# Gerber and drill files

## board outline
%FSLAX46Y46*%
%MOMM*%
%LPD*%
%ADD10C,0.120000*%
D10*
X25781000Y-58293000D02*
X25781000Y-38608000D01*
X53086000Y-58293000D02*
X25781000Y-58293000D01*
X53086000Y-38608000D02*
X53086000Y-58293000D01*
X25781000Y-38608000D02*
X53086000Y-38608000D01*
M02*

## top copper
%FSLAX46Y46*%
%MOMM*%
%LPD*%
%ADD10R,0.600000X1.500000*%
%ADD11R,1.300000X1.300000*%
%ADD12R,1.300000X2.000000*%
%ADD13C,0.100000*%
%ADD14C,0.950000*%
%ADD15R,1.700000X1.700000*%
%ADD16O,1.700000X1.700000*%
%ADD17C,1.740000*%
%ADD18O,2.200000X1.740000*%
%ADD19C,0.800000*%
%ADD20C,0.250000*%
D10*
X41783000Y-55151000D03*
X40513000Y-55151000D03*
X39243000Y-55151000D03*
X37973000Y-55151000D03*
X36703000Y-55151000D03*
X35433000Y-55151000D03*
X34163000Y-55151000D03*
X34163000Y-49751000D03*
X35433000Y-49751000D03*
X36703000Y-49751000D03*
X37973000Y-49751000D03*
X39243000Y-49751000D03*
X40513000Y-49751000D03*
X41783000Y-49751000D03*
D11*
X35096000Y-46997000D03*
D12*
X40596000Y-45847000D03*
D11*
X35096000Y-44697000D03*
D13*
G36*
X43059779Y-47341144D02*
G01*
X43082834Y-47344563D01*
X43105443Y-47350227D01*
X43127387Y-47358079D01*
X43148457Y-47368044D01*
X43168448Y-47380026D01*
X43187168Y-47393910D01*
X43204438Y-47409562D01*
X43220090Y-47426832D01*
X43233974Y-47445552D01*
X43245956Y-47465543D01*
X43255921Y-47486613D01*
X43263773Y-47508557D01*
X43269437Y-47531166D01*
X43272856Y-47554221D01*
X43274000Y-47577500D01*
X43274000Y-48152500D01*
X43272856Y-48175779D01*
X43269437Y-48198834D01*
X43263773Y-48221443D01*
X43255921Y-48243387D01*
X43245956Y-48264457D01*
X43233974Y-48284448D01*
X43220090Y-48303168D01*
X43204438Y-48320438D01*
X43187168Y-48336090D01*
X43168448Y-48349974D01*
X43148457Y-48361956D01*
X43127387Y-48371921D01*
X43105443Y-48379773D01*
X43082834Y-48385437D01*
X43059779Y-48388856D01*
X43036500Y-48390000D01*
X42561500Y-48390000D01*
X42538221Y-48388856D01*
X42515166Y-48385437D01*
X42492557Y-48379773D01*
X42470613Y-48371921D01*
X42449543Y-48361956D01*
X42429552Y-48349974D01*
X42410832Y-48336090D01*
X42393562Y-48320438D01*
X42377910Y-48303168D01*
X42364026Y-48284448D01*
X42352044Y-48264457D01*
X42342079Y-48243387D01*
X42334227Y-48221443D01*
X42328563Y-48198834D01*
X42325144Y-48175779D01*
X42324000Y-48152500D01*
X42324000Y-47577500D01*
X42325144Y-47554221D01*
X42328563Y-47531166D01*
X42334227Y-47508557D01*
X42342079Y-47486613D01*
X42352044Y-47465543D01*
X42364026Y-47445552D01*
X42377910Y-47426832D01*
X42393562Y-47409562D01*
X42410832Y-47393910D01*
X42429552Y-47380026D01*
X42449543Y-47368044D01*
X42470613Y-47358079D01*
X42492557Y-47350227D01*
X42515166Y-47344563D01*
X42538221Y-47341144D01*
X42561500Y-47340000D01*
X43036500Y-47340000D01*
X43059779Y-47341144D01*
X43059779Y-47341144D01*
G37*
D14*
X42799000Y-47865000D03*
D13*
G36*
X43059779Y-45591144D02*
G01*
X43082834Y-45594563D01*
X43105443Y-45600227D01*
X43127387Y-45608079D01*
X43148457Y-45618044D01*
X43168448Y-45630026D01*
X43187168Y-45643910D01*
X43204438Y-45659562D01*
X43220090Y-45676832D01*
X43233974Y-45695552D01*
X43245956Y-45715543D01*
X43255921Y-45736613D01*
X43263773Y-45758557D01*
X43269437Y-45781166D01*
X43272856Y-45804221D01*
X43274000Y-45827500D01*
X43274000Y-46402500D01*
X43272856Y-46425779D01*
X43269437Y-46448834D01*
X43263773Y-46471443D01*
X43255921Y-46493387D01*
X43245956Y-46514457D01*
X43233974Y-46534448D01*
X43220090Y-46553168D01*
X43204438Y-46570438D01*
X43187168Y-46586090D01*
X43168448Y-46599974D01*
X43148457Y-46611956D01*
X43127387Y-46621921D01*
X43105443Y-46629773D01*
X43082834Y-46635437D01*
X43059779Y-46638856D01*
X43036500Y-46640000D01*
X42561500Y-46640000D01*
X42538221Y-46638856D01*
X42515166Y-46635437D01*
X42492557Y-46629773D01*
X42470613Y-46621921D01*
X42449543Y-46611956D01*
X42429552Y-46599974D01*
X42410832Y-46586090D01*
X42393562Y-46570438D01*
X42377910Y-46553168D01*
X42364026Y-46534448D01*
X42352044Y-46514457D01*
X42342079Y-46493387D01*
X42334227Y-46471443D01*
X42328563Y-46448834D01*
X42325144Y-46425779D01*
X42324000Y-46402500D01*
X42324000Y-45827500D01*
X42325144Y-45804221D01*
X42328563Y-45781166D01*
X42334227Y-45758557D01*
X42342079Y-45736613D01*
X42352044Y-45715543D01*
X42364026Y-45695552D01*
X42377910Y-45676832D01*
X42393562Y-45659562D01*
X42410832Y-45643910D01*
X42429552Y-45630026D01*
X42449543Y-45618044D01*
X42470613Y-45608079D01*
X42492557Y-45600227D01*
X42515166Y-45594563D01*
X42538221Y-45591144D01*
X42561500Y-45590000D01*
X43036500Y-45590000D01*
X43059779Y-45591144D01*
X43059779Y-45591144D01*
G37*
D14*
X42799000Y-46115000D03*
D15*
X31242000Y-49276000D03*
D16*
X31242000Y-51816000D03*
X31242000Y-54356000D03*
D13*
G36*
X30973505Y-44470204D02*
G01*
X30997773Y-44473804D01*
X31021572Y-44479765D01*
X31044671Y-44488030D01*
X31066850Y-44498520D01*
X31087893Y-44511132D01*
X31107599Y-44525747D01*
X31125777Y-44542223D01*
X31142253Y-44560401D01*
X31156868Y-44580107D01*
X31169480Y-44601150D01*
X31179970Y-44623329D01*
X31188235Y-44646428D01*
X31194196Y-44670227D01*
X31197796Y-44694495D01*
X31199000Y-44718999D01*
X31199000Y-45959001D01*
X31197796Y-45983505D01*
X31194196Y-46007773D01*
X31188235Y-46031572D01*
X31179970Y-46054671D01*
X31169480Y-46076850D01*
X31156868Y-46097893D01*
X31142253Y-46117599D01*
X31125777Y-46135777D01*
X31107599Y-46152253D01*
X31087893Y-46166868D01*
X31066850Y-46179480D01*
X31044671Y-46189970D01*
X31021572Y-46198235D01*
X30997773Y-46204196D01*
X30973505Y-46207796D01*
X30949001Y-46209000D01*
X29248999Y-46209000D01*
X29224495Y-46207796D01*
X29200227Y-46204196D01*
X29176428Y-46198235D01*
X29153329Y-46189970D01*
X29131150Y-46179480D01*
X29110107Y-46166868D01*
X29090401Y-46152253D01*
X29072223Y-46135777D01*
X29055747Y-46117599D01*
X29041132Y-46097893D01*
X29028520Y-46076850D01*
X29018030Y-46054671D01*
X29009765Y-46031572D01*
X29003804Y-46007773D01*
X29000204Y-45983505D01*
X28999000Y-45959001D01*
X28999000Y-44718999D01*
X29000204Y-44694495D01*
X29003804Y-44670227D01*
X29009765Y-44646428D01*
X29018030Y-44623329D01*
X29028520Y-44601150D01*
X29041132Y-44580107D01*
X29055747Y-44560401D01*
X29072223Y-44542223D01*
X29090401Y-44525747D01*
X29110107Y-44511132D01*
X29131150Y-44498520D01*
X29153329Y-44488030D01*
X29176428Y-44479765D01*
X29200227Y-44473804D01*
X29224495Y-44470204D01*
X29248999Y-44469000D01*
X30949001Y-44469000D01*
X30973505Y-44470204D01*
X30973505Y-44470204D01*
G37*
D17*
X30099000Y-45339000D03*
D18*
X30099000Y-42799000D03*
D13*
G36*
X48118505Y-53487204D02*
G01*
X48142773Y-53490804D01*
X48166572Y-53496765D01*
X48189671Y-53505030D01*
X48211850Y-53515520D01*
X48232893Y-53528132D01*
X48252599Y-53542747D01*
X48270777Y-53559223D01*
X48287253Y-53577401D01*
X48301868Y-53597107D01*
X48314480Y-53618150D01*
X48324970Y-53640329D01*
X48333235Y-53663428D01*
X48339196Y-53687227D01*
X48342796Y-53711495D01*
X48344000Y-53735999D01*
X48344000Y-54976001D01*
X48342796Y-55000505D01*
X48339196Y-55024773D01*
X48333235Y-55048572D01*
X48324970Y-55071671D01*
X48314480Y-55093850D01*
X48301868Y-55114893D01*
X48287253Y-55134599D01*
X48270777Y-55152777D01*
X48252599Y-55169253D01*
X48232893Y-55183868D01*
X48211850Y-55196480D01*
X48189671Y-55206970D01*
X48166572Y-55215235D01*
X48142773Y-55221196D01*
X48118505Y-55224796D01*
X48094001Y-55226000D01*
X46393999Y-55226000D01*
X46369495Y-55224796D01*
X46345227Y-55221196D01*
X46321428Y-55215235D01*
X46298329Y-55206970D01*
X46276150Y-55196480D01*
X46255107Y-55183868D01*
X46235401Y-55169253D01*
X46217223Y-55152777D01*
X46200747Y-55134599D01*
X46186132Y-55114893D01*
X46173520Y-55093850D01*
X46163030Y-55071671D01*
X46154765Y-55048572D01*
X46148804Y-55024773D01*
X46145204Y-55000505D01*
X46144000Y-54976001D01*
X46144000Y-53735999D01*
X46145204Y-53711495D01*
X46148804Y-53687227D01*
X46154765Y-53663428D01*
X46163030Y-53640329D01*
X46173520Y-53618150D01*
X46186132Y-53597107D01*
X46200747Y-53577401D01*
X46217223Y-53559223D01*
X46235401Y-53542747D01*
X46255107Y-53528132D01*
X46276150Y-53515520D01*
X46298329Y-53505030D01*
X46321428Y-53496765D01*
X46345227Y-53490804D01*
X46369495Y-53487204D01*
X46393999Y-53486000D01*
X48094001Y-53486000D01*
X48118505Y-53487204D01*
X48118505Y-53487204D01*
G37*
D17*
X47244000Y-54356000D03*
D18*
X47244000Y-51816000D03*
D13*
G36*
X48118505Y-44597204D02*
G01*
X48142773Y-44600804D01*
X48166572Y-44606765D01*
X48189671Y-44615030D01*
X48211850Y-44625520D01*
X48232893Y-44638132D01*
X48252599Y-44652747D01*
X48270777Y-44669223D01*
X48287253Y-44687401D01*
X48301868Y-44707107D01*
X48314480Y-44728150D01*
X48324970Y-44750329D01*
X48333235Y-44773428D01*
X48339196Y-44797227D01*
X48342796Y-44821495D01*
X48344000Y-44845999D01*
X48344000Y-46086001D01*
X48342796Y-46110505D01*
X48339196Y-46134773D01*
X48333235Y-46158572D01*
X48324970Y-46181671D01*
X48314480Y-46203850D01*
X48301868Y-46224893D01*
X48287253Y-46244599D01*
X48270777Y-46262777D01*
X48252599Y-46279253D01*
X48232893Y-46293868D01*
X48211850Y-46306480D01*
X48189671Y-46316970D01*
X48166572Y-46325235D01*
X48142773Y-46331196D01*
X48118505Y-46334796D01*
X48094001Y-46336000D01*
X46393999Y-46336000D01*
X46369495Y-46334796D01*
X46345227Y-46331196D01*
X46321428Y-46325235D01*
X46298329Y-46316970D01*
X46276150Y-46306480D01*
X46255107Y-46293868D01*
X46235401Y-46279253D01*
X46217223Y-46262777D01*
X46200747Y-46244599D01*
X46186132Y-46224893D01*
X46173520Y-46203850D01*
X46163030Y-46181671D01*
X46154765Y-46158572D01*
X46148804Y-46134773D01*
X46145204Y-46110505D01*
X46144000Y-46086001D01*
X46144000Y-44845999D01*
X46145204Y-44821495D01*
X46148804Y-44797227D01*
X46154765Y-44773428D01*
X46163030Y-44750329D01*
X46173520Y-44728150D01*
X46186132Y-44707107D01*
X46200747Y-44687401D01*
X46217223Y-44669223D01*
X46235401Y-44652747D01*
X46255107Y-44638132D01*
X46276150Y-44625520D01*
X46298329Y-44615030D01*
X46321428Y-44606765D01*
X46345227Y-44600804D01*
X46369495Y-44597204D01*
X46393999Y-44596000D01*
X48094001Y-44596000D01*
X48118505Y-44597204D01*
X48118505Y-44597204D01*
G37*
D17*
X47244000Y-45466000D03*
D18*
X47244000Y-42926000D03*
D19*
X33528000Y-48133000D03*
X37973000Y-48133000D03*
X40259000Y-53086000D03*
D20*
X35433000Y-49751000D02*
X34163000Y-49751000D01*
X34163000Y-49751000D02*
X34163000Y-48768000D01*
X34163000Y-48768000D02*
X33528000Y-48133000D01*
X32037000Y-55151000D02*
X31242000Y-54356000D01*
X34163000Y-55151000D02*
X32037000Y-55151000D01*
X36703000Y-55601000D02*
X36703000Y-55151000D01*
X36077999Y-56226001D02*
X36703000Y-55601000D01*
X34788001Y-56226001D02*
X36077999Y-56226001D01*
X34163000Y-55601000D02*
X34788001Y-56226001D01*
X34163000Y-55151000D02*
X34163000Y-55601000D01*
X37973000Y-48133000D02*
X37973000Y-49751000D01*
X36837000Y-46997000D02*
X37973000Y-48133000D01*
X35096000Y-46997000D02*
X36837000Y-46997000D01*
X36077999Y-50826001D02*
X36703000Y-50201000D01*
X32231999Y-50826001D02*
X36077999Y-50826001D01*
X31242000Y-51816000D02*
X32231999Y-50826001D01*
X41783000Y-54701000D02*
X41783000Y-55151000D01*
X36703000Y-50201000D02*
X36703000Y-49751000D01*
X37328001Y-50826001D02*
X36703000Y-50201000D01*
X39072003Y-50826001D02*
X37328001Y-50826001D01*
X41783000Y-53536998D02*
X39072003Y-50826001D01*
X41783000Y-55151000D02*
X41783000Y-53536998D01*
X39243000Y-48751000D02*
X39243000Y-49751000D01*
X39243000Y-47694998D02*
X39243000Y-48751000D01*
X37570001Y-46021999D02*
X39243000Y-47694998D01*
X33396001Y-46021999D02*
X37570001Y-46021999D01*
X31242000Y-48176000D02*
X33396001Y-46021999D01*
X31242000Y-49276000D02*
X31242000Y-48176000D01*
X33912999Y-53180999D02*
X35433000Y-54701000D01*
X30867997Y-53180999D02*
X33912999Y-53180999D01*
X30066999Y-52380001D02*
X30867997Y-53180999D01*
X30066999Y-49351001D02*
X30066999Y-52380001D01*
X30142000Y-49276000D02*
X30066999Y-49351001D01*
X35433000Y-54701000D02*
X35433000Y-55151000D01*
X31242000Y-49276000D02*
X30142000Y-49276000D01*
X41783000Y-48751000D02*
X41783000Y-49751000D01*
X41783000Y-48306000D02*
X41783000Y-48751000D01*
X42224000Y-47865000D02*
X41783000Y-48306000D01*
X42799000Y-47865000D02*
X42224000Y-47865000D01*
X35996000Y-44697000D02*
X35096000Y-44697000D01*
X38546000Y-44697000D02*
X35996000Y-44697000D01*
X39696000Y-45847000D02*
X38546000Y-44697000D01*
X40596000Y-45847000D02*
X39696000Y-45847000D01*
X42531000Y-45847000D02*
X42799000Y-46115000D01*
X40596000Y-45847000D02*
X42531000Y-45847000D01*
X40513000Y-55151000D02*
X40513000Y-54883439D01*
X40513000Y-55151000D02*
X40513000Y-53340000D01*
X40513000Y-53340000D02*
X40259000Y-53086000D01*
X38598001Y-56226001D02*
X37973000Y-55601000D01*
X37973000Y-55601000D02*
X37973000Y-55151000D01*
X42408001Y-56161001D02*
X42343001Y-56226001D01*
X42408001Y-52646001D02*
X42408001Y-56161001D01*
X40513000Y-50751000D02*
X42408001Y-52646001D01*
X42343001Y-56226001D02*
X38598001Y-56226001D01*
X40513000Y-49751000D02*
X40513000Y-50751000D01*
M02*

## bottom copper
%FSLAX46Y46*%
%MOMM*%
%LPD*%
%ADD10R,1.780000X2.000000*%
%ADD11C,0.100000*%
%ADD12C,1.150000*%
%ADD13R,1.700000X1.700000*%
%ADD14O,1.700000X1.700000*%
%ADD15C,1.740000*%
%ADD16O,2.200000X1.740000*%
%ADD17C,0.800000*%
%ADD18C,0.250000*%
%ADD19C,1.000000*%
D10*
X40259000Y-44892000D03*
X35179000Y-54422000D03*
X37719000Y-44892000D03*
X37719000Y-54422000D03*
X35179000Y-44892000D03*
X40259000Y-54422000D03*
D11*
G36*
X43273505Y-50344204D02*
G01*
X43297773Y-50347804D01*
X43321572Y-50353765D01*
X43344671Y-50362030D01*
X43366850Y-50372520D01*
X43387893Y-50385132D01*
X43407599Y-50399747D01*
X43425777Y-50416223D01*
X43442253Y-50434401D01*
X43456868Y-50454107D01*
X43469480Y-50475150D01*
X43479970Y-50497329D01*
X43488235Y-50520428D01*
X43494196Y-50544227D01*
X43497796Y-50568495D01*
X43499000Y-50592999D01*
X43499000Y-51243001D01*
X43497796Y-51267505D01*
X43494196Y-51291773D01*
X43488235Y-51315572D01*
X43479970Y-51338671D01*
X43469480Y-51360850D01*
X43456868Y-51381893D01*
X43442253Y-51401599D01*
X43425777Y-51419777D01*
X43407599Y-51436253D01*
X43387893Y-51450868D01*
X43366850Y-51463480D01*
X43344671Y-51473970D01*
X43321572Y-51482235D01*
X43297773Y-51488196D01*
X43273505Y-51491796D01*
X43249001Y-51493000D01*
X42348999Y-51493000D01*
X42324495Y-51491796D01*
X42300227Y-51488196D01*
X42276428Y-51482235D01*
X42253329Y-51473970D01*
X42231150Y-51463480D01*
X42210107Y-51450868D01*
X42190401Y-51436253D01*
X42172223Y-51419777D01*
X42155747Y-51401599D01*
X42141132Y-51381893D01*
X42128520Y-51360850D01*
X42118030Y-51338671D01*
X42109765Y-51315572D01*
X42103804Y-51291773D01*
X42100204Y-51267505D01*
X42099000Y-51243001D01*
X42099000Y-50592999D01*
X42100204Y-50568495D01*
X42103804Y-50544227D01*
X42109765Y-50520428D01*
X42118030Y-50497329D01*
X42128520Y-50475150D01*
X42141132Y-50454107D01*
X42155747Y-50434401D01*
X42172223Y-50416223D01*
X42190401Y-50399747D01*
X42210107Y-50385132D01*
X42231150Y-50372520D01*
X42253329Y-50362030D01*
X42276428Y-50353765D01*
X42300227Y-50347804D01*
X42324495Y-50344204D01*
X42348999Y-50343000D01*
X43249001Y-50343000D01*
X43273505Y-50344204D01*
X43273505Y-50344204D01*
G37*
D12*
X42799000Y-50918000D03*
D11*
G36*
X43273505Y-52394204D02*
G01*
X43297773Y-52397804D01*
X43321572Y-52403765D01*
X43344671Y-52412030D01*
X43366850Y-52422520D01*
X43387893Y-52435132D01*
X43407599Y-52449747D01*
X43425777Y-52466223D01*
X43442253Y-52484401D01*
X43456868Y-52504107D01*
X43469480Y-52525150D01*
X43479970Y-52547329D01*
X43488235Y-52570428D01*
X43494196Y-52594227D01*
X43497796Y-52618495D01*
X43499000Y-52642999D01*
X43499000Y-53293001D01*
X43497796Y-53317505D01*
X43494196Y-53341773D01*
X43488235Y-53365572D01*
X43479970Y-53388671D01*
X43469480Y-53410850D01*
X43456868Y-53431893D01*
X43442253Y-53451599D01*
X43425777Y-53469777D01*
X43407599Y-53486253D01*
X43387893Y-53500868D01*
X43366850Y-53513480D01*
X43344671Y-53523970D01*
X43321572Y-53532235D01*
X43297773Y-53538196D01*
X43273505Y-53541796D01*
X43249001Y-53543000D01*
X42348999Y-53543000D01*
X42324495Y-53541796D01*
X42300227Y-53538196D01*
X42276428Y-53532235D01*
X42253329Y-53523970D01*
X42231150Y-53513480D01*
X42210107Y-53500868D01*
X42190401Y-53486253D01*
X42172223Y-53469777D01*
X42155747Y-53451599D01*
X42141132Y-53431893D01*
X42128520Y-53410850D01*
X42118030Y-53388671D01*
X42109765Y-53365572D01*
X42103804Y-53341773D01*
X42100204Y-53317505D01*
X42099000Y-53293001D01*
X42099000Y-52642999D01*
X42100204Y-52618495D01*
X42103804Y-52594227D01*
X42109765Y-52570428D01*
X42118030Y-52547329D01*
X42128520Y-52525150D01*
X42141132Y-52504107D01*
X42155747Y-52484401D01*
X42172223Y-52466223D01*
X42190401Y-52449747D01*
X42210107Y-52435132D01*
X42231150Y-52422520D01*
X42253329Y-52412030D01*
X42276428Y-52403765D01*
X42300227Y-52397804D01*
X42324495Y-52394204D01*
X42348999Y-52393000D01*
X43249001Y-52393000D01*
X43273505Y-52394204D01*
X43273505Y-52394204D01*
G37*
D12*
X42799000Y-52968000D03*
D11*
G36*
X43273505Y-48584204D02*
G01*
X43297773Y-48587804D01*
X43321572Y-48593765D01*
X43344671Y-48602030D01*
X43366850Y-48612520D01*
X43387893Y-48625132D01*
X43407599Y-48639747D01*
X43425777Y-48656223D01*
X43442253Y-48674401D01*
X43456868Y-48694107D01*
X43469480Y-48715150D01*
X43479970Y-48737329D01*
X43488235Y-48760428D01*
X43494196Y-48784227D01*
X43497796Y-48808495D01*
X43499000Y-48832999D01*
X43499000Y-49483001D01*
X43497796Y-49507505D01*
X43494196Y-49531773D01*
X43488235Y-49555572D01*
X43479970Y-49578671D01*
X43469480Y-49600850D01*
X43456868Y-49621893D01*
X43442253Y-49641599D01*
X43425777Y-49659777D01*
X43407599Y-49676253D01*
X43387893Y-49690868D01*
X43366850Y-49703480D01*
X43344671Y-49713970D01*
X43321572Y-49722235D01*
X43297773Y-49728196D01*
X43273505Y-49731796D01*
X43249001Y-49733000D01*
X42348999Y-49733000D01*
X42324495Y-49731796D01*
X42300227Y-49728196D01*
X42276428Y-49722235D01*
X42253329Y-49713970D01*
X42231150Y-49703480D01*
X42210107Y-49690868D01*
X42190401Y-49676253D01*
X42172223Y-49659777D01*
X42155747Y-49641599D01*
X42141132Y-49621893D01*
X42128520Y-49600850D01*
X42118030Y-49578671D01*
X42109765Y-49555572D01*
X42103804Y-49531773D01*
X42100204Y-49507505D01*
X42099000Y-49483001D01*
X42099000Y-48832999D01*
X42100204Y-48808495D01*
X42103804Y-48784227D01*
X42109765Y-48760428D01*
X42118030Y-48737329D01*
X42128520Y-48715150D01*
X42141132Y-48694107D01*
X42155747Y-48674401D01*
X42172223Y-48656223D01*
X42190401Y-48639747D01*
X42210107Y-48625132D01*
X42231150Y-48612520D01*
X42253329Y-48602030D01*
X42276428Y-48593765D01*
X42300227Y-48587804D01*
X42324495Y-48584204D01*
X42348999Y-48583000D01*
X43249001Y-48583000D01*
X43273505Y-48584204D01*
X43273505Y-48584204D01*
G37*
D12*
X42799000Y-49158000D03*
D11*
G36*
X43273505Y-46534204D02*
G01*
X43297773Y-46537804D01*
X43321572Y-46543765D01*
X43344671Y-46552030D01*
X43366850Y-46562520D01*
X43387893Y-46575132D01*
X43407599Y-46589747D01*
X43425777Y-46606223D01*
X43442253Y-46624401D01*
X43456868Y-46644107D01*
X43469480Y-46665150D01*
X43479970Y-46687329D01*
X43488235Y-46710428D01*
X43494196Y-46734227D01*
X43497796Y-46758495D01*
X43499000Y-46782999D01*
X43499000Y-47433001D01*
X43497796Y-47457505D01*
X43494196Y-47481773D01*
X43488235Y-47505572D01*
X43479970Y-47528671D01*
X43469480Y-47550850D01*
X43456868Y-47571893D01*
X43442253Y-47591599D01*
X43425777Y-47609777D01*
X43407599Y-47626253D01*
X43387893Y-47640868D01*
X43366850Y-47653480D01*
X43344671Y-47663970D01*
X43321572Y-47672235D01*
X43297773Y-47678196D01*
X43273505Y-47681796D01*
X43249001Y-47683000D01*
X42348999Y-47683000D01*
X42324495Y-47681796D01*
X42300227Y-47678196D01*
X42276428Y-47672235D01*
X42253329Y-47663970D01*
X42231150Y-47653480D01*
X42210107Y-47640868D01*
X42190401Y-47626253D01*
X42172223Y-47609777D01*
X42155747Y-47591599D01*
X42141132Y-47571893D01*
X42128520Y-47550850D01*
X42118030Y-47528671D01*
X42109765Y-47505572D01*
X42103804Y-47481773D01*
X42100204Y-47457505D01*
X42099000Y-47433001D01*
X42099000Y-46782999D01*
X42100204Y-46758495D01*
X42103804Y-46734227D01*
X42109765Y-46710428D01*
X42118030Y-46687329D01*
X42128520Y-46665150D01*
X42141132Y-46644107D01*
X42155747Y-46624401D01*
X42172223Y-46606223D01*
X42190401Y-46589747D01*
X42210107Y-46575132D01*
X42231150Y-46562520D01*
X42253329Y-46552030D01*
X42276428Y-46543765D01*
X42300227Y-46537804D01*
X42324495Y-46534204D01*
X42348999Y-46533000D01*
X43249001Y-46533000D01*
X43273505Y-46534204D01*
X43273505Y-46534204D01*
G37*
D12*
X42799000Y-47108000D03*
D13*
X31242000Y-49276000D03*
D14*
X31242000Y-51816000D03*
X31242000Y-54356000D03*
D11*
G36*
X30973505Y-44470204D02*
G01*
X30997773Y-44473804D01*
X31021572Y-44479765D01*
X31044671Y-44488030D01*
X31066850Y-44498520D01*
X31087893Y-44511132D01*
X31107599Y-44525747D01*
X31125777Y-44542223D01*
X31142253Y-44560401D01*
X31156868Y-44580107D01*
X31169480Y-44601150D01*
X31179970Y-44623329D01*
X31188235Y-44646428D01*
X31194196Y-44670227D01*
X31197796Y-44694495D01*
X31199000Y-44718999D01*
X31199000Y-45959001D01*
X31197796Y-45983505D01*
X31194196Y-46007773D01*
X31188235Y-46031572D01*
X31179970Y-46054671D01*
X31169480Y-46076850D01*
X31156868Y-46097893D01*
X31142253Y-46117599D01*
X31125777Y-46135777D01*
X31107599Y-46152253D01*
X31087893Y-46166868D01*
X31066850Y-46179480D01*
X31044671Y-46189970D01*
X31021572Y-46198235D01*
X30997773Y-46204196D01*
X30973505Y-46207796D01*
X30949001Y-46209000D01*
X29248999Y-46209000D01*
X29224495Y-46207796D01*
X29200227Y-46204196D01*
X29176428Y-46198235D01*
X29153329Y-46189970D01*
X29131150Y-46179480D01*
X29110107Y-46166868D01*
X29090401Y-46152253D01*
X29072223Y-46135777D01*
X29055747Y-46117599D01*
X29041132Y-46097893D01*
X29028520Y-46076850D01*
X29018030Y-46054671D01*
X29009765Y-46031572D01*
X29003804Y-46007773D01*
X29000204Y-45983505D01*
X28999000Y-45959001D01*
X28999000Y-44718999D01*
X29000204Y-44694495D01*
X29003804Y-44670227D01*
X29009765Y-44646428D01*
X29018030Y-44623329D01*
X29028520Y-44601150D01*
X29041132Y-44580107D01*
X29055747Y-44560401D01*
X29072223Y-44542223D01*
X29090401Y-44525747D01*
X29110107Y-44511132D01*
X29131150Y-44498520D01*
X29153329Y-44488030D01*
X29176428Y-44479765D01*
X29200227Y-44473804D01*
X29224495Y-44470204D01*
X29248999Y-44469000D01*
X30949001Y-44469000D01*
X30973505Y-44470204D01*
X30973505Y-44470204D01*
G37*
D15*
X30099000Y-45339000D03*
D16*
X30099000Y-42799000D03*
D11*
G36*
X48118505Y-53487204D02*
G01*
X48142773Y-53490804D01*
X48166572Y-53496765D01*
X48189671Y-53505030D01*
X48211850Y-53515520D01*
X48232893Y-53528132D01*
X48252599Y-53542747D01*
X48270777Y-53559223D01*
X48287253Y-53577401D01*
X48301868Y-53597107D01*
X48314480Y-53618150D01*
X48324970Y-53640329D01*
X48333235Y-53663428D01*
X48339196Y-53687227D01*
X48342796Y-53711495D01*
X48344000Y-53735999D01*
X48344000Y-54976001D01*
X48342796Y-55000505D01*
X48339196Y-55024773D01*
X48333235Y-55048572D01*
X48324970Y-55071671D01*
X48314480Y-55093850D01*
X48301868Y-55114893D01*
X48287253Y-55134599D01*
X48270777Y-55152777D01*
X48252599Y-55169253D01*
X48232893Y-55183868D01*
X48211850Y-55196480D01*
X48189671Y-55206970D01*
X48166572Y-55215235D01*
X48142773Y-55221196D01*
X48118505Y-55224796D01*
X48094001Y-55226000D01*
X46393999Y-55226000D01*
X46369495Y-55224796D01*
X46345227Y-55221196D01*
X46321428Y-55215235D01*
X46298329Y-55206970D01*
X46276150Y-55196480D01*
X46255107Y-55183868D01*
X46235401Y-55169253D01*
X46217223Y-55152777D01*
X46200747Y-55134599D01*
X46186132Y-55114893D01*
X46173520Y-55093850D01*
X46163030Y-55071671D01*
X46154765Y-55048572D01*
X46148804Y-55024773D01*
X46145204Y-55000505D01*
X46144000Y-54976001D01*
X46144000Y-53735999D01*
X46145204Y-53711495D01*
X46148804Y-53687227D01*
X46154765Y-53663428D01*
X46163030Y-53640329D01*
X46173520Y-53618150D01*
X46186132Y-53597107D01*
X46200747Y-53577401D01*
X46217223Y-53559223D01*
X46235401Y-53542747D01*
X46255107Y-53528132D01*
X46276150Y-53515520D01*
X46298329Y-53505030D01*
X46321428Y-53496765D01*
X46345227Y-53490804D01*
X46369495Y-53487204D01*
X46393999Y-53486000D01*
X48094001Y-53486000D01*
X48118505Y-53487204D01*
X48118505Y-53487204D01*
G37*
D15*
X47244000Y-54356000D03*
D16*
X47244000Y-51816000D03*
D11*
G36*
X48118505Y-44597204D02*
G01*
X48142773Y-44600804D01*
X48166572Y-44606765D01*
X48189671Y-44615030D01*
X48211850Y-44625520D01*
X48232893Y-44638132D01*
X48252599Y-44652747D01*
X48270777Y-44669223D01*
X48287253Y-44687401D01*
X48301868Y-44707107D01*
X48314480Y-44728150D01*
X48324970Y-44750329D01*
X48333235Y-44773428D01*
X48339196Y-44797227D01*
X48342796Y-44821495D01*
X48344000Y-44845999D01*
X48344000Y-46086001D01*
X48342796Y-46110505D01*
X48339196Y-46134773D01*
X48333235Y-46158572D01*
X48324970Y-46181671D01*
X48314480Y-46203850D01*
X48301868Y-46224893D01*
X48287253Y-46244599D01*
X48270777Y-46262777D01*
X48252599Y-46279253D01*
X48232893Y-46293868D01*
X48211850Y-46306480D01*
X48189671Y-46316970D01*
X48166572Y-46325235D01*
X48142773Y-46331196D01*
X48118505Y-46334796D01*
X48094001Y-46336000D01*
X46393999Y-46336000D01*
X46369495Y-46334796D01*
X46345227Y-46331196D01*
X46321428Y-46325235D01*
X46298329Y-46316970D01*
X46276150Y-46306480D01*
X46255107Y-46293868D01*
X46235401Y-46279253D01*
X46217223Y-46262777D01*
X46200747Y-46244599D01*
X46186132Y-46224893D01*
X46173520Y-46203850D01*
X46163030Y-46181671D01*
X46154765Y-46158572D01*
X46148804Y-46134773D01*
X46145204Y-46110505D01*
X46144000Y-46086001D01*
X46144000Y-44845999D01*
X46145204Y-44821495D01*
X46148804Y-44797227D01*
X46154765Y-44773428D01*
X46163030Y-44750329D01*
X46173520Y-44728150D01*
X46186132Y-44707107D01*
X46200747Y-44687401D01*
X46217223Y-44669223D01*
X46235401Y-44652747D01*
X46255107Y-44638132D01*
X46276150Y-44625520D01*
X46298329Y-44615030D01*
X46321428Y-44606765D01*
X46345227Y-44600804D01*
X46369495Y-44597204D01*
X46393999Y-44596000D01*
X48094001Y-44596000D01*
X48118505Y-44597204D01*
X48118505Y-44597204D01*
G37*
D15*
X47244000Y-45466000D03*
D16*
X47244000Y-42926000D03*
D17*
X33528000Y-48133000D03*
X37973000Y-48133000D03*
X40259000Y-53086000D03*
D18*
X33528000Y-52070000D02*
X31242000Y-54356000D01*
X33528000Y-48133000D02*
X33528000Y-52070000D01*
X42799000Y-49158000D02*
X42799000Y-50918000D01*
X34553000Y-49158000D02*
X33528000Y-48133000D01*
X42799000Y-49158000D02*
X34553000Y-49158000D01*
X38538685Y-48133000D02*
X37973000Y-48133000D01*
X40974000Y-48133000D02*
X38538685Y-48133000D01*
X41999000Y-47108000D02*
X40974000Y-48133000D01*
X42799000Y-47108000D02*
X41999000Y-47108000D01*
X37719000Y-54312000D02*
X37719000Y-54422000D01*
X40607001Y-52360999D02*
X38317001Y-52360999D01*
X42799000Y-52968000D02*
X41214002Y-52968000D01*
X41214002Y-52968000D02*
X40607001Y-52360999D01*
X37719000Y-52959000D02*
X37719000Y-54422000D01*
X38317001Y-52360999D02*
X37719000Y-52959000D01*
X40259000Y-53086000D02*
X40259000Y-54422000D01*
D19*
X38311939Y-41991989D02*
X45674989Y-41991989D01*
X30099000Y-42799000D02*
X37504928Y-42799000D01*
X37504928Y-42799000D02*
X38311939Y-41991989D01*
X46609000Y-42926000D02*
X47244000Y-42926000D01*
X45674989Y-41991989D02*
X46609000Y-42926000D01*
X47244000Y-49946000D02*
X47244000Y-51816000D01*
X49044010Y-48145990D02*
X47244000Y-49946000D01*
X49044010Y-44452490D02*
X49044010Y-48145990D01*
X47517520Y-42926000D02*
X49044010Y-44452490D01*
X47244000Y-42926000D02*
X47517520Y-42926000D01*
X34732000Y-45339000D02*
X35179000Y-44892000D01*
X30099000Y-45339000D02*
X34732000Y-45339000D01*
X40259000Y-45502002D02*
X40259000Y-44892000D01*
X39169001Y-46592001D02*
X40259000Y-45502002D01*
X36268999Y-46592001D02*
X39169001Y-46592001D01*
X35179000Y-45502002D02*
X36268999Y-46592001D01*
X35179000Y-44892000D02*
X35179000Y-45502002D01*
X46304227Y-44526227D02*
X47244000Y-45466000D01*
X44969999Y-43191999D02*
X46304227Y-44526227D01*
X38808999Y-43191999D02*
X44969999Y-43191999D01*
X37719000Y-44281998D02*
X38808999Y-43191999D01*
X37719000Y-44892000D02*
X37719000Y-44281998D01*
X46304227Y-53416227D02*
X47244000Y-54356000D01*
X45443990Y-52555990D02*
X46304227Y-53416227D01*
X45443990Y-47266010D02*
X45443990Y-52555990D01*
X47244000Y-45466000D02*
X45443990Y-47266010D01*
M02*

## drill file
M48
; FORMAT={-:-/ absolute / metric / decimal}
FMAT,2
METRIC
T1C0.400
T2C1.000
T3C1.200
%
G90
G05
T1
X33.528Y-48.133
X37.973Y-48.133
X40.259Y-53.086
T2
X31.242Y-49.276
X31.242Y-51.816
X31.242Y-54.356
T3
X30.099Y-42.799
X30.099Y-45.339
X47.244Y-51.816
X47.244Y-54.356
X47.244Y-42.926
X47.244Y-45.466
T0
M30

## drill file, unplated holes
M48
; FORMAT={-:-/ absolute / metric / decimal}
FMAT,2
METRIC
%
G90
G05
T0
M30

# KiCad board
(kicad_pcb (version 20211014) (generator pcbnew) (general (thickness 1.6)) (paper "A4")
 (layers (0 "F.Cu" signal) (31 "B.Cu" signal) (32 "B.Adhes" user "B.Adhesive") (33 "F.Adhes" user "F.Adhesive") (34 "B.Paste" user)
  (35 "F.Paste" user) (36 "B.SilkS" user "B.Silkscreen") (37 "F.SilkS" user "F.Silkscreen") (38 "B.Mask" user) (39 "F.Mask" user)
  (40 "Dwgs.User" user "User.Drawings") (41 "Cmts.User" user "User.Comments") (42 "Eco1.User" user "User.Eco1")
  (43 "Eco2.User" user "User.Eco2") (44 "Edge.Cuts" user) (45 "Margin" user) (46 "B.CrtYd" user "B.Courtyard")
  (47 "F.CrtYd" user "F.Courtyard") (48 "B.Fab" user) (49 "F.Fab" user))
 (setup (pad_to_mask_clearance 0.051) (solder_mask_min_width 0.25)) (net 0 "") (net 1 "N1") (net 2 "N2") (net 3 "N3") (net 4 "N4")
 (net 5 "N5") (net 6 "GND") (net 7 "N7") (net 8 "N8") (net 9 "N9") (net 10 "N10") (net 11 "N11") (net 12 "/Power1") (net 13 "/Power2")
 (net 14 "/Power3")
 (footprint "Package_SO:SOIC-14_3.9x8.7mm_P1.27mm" (layer "F.Cu") (at 37.973 52.451 -90)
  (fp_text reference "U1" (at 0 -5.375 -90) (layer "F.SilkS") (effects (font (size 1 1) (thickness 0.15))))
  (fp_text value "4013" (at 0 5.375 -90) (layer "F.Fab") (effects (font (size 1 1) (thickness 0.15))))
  (pad "1" smd rect locked (at -2.7 -3.81 270) (size 1.5 0.6) (layers "F.Cu" "F.Paste" "F.Mask") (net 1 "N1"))
  (pad "2" smd rect locked (at -2.7 -2.54 270) (size 1.5 0.6) (layers "F.Cu" "F.Paste" "F.Mask") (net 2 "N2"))
  (pad "3" smd rect locked (at -2.7 -1.27 270) (size 1.5 0.6) (layers "F.Cu" "F.Paste" "F.Mask") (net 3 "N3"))
  (pad "4" smd rect locked (at -2.7 0 270) (size 1.5 0.6) (layers "F.Cu" "F.Paste" "F.Mask") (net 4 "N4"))
  (pad "5" smd rect locked (at -2.7 1.27 270) (size 1.5 0.6) (layers "F.Cu" "F.Paste" "F.Mask") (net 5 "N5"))
  (pad "6" smd rect locked (at -2.7 2.54 270) (size 1.5 0.6) (layers "F.Cu" "F.Paste" "F.Mask") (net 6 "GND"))
  (pad "7" smd rect locked (at -2.7 3.81 270) (size 1.5 0.6) (layers "F.Cu" "F.Paste" "F.Mask") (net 6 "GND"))
  (pad "8" smd rect locked (at 2.7 3.81 270) (size 1.5 0.6) (layers "F.Cu" "F.Paste" "F.Mask") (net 6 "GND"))
  (pad "9" smd rect locked (at 2.7 2.54 270) (size 1.5 0.6) (layers "F.Cu" "F.Paste" "F.Mask") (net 3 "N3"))
  (pad "10" smd rect locked (at 2.7 1.27 270) (size 1.5 0.6) (layers "F.Cu" "F.Paste" "F.Mask") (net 6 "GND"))
  (pad "11" smd rect locked (at 2.7 0 270) (size 1.5 0.6) (layers "F.Cu" "F.Paste" "F.Mask") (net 2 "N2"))
  (pad "12" smd rect locked (at 2.7 -1.27 270) (size 1.5 0.6) (layers "F.Cu" "F.Paste" "F.Mask") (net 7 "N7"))
  (pad "13" smd rect locked (at 2.7 -2.54 270) (size 1.5 0.6) (layers "F.Cu" "F.Paste" "F.Mask") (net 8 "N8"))
  (pad "14" smd rect locked (at 2.7 -3.81 270) (size 1.5 0.6) (layers "F.Cu" "F.Paste" "F.Mask") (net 5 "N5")))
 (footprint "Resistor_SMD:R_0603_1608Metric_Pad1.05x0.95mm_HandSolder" (layer "F.Cu") (at 42.799 46.99 -90)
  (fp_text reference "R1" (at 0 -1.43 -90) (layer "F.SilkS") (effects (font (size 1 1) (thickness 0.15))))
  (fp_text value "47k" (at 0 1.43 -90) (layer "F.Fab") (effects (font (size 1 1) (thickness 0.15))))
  (pad "1" smd roundrect locked (at -0.875 0 270) (size 1.05 0.95) (layers "F.Cu" "F.Paste" "F.Mask") (roundrect_rratio 0.25) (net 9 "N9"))
  (pad "2" smd roundrect locked (at 0.875 0 270) (size 1.05 0.95) (layers "F.Cu" "F.Paste" "F.Mask") (roundrect_rratio 0.25) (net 1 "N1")))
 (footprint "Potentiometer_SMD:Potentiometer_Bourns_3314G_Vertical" (layer "F.Cu") (at 37.846 45.847 90)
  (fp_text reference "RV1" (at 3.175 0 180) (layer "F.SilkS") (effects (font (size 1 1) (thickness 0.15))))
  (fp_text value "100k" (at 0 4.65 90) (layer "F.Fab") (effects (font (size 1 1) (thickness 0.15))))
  (pad "1" smd rect locked (at 1.15 -2.75 90) (size 1.3 1.3) (layers "F.Cu" "F.Paste" "F.Mask") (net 9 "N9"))
  (pad "2" smd rect locked (at 0 2.75 90) (size 2 1.3) (layers "F.Cu" "F.Paste" "F.Mask") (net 9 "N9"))
  (pad "3" smd rect locked (at -1.15 -2.75 90) (size 1.3 1.3) (layers "F.Cu" "F.Paste" "F.Mask") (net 4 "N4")))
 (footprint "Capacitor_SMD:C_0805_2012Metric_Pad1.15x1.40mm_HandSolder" (layer "B.Cu") (at 42.799 48.133 -90)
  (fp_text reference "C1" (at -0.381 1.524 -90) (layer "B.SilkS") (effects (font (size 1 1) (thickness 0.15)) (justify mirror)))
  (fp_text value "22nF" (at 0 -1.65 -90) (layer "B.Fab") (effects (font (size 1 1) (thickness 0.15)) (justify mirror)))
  (pad "1" smd roundrect locked (at -1.025 0 270) (size 1.15 1.4) (layers "B.Cu" "B.Paste" "B.Mask") (roundrect_rratio 0.217391)
   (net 4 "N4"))
  (pad "2" smd roundrect locked (at 1.025 0 270) (size 1.15 1.4) (layers "B.Cu" "B.Paste" "B.Mask") (roundrect_rratio 0.217391)
   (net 6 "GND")))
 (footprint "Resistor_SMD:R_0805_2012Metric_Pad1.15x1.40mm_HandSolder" (layer "B.Cu") (at 42.799 51.943 90)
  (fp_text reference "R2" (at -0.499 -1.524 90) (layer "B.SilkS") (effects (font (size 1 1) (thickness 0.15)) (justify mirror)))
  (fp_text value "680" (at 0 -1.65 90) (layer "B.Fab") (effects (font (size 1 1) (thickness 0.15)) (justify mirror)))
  (pad "1" smd roundrect locked (at -1.025 0 90) (size 1.15 1.4) (layers "B.Cu" "B.Paste" "B.Mask") (roundrect_rratio 0.217391)
   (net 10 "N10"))
  (pad "2" smd roundrect locked (at 1.025 0 90) (size 1.15 1.4) (layers "B.Cu" "B.Paste" "B.Mask") (roundrect_rratio 0.217391) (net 6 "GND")))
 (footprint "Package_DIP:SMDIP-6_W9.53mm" (layer "B.Cu") (at 37.719 49.657 90)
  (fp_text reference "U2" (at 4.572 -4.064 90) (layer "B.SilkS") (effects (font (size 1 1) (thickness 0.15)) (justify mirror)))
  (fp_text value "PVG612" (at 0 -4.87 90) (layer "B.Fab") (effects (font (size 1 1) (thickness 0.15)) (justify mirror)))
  (pad "1" smd rect locked (at -4.765 2.54 90) (size 2 1.78) (layers "B.Cu" "B.Paste" "B.Mask") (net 8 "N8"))
  (pad "2" smd rect locked (at -4.765 0 90) (size 2 1.78) (layers "B.Cu" "B.Paste" "B.Mask") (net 10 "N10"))
  (pad "3" smd rect locked (at -4.765 -2.54 90) (size 2 1.78) (layers "B.Cu" "B.Paste" "B.Mask") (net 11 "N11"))
  (pad "4" smd rect locked (at 4.765 -2.54 90) (size 2 1.78) (layers "B.Cu" "B.Paste" "B.Mask") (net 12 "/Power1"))
  (pad "5" smd rect locked (at 4.765 0 90) (size 2 1.78) (layers "B.Cu" "B.Paste" "B.Mask") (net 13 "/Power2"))
  (pad "6" smd rect locked (at 4.765 2.54 90) (size 2 1.78) (layers "B.Cu" "B.Paste" "B.Mask") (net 12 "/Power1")))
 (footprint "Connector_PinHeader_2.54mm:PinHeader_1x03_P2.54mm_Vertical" (layer "B.Cu") (at 31.242 49.276 180)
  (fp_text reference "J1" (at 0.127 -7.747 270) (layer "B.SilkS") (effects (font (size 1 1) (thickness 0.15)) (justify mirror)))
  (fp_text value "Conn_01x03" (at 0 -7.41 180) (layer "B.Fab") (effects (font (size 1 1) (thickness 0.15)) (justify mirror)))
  (pad "1" thru_hole rect locked (at 0 0 180) (size 1.7 1.7) (drill 1) (layers *.Cu *.Mask) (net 3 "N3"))
  (pad "2" thru_hole oval locked (at 0 -2.54 180) (size 1.7 1.7) (drill 1) (layers *.Cu *.Mask) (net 5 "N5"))
  (pad "3" thru_hole oval locked (at 0 -5.08 180) (size 1.7 1.7) (drill 1) (layers *.Cu *.Mask) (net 6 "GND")))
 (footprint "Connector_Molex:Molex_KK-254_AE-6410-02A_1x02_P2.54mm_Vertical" (layer "B.Cu") (at 30.099 45.339 90)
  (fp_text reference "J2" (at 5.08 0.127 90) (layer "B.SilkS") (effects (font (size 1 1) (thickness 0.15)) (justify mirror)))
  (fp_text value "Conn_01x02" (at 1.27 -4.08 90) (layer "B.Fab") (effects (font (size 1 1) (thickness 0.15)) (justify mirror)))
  (pad "1" thru_hole roundrect locked (at 0 0 90) (size 1.74 2.2) (drill 1.2) (layers *.Cu *.Mask) (roundrect_rratio 0.143678)
   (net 12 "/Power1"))
  (pad "2" thru_hole oval locked (at 2.54 0 90) (size 1.74 2.2) (drill 1.2) (layers *.Cu *.Mask) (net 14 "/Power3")))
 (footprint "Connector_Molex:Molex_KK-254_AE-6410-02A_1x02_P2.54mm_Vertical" (layer "B.Cu") (at 47.244 54.356 90)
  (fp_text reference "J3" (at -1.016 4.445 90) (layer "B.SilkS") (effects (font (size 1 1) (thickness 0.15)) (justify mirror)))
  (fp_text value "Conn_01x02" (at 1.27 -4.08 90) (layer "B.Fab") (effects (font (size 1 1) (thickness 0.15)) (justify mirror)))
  (pad "1" thru_hole roundrect locked (at 0 0 90) (size 1.74 2.2) (drill 1.2) (layers *.Cu *.Mask) (roundrect_rratio 0.143678)
   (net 13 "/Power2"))
  (pad "2" thru_hole oval locked (at 2.54 0 90) (size 1.74 2.2) (drill 1.2) (layers *.Cu *.Mask) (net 14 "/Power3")))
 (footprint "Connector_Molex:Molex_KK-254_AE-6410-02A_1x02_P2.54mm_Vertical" (layer "B.Cu") (at 47.244 45.466 90)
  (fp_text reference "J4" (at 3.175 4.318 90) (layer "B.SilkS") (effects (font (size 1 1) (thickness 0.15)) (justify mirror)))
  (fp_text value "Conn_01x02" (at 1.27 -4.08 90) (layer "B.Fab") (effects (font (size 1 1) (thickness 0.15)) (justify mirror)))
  (pad "1" thru_hole roundrect locked (at 0 0 90) (size 1.74 2.2) (drill 1.2) (layers *.Cu *.Mask) (roundrect_rratio 0.143678)
   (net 13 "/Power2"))
  (pad "2" thru_hole oval locked (at 2.54 0 90) (size 1.74 2.2) (drill 1.2) (layers *.Cu *.Mask) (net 14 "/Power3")))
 (gr_line (start 25.781 58.293) (end 25.781 38.608) (layer "Edge.Cuts") (width 0.12))
 (gr_line (start 25.781 38.608) (end 53.086 38.608) (layer "Edge.Cuts") (width 0.12))
 (gr_line (start 53.086 38.608) (end 53.086 58.293) (layer "Edge.Cuts") (width 0.12))
 (gr_line (start 53.086 58.293) (end 25.781 58.293) (layer "Edge.Cuts") (width 0.12))
 (segment (start 34.163 55.151) (end 34.163 55.601) (width 0.25) (layer "F.Cu") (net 6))
 (segment (start 34.163 48.768) (end 33.528 48.133) (width 0.25) (layer "F.Cu") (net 6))
 (segment (start 34.163 55.151) (end 32.037 55.151) (width 0.25) (layer "F.Cu") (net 6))
 (segment (start 36.077999 56.226001) (end 36.703 55.601) (width 0.25) (layer "F.Cu") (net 6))
 (segment (start 34.163 55.601) (end 34.788001 56.226001) (width 0.25) (layer "F.Cu") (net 6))
 (segment (start 35.433 49.751) (end 34.163 49.751) (width 0.25) (layer "F.Cu") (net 6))
 (segment (start 32.037 55.151) (end 31.242 54.356) (width 0.25) (layer "F.Cu") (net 6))
 (segment (start 34.163 49.751) (end 34.163 48.768) (width 0.25) (layer "F.Cu") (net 6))
 (segment (start 36.703 55.601) (end 36.703 55.151) (width 0.25) (layer "F.Cu") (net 6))
 (segment (start 34.788001 56.226001) (end 36.077999 56.226001) (width 0.25) (layer "F.Cu") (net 6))
 (via (at 33.528 48.133) (size 0.8) (drill 0.4) (layers "F.Cu" "B.Cu") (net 6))
 (segment (start 42.799 49.158) (end 42.799 50.918) (width 0.25) (layer "B.Cu") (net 6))
 (segment (start 34.553 49.158) (end 33.528 48.133) (width 0.25) (layer "B.Cu") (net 6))
 (segment (start 33.528 48.133) (end 33.528 52.07) (width 0.25) (layer "B.Cu") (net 6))
 (segment (start 33.528 52.07) (end 31.242 54.356) (width 0.25) (layer "B.Cu") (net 6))
 (segment (start 42.799 49.158) (end 34.553 49.158) (width 0.25) (layer "B.Cu") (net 6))
 (segment (start 35.096 46.997) (end 36.837 46.997) (width 0.25) (layer "F.Cu") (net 4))
 (segment (start 36.837 46.997) (end 37.973 48.133) (width 0.25) (layer "F.Cu") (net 4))
 (segment (start 37.973 48.133) (end 37.973 49.751) (width 0.25) (layer "F.Cu") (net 4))
 (via (at 37.973 48.133) (size 0.8) (drill 0.4) (layers "F.Cu" "B.Cu") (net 4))
 (segment (start 41.999 47.108) (end 40.974 48.133) (width 0.25) (layer "B.Cu") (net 4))
 (segment (start 40.974 48.133) (end 38.538685 48.133) (width 0.25) (layer "B.Cu") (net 4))
 (segment (start 38.538685 48.133) (end 37.973 48.133) (width 0.25) (layer "B.Cu") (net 4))
 (segment (start 42.799 47.108) (end 41.999 47.108) (width 0.25) (layer "B.Cu") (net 4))
 (segment (start 36.703 50.201) (end 36.703 49.751) (width 0.25) (layer "F.Cu") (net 5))
 (segment (start 41.783 55.151) (end 41.783 53.536998) (width 0.25) (layer "F.Cu") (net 5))
 (segment (start 31.242 51.816) (end 32.231999 50.826001) (width 0.25) (layer "F.Cu") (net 5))
 (segment (start 36.077999 50.826001) (end 36.703 50.201) (width 0.25) (layer "F.Cu") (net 5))
 (segment (start 32.231999 50.826001) (end 36.077999 50.826001) (width 0.25) (layer "F.Cu") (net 5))
 (segment (start 37.328001 50.826001) (end 36.703 50.201) (width 0.25) (layer "F.Cu") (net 5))
 (segment (start 41.783 54.701) (end 41.783 55.151) (width 0.25) (layer "F.Cu") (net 5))
 (segment (start 39.072003 50.826001) (end 37.328001 50.826001) (width 0.25) (layer "F.Cu") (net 5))
 (segment (start 41.783 53.536998) (end 39.072003 50.826001) (width 0.25) (layer "F.Cu") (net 5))
 (segment (start 37.570001 46.021999) (end 39.243 47.694998) (width 0.25) (layer "F.Cu") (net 3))
 (segment (start 30.142 49.276) (end 30.066999 49.351001) (width 0.25) (layer "F.Cu") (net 3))
 (segment (start 31.242 49.276) (end 30.142 49.276) (width 0.25) (layer "F.Cu") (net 3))
 (segment (start 35.433 54.701) (end 35.433 55.151) (width 0.25) (layer "F.Cu") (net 3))
 (segment (start 39.243 47.694998) (end 39.243 48.751) (width 0.25) (layer "F.Cu") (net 3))
 (segment (start 31.242 49.276) (end 31.242 48.176) (width 0.25) (layer "F.Cu") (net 3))
 (segment (start 30.066999 52.380001) (end 30.867997 53.180999) (width 0.25) (layer "F.Cu") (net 3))
 (segment (start 39.243 48.751) (end 39.243 49.751) (width 0.25) (layer "F.Cu") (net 3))
 (segment (start 30.867997 53.180999) (end 33.912999 53.180999) (width 0.25) (layer "F.Cu") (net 3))
 (segment (start 33.396001 46.021999) (end 37.570001 46.021999) (width 0.25) (layer "F.Cu") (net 3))
 (segment (start 31.242 48.176) (end 33.396001 46.021999) (width 0.25) (layer "F.Cu") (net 3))
 (segment (start 33.912999 53.180999) (end 35.433 54.701) (width 0.25) (layer "F.Cu") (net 3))
 (segment (start 30.066999 49.351001) (end 30.066999 52.380001) (width 0.25) (layer "F.Cu") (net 3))
 (segment (start 42.224 47.865) (end 41.783 48.306) (width 0.25) (layer "F.Cu") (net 1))
 (segment (start 41.783 48.751) (end 41.783 49.751) (width 0.25) (layer "F.Cu") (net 1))
 (segment (start 42.799 47.865) (end 42.224 47.865) (width 0.25) (layer "F.Cu") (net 1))
 (segment (start 41.783 48.306) (end 41.783 48.751) (width 0.25) (layer "F.Cu") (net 1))
 (segment (start 39.696 45.847) (end 38.546 44.697) (width 0.25) (layer "F.Cu") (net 9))
 (segment (start 40.596 45.847) (end 39.696 45.847) (width 0.25) (layer "F.Cu") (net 9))
 (segment (start 42.531 45.847) (end 42.799 46.115) (width 0.25) (layer "F.Cu") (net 9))
 (segment (start 35.996 44.697) (end 35.096 44.697) (width 0.25) (layer "F.Cu") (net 9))
 (segment (start 40.596 45.847) (end 42.531 45.847) (width 0.25) (layer "F.Cu") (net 9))
 (segment (start 38.546 44.697) (end 35.996 44.697) (width 0.25) (layer "F.Cu") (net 9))
 (segment (start 38.317001 52.360999) (end 37.719 52.959) (width 0.25) (layer "B.Cu") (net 10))
 (segment (start 41.214002 52.968) (end 40.607001 52.360999) (width 0.25) (layer "B.Cu") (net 10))
 (segment (start 37.719 52.959) (end 37.719 54.422) (width 0.25) (layer "B.Cu") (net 10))
 (segment (start 40.607001 52.360999) (end 38.317001 52.360999) (width 0.25) (layer "B.Cu") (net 10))
 (segment (start 42.799 52.968) (end 41.214002 52.968) (width 0.25) (layer "B.Cu") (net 10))
 (segment (start 37.719 54.312) (end 37.719 54.422) (width 0.25) (layer "B.Cu") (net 10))
 (segment (start 40.513 53.34) (end 40.259 53.086) (width 0.25) (layer "F.Cu") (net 8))
 (segment (start 40.513 55.151) (end 40.513 54.883439) (width 0.25) (layer "F.Cu") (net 8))
 (segment (start 40.513 55.151) (end 40.513 53.34) (width 0.25) (layer "F.Cu") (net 8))
 (via (at 40.259 53.086) (size 0.8) (drill 0.4) (layers "F.Cu" "B.Cu") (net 8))
 (segment (start 40.259 53.086) (end 40.259 54.422) (width 0.25) (layer "B.Cu") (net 8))
 (segment (start 42.408001 56.161001) (end 42.343001 56.226001) (width 0.25) (layer "F.Cu") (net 2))
 (segment (start 40.513 49.751) (end 40.513 50.751) (width 0.25) (layer "F.Cu") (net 2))
 (segment (start 42.408001 52.646001) (end 42.408001 56.161001) (width 0.25) (layer "F.Cu") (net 2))
 (segment (start 38.598001 56.226001) (end 37.973 55.601) (width 0.25) (layer "F.Cu") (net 2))
 (segment (start 40.513 50.751) (end 42.408001 52.646001) (width 0.25) (layer "F.Cu") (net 2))
 (segment (start 37.973 55.601) (end 37.973 55.151) (width 0.25) (layer "F.Cu") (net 2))
 (segment (start 42.343001 56.226001) (end 38.598001 56.226001) (width 0.25) (layer "F.Cu") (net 2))
 (segment (start 45.674989 41.991989) (end 46.609 42.926) (width 1) (layer "B.Cu") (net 14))
 (segment (start 38.311939 41.991989) (end 45.674989 41.991989) (width 1) (layer "B.Cu") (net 14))
 (segment (start 30.099 42.799) (end 37.504928 42.799) (width 1) (layer "B.Cu") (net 14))
 (segment (start 46.609 42.926) (end 47.244 42.926) (width 1) (layer "B.Cu") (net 14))
 (segment (start 49.04401 44.45249) (end 49.04401 48.14599) (width 1) (layer "B.Cu") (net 14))
 (segment (start 49.04401 48.14599) (end 47.244 49.946) (width 1) (layer "B.Cu") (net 14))
 (segment (start 37.504928 42.799) (end 38.311939 41.991989) (width 1) (layer "B.Cu") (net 14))
 (segment (start 47.244 49.946) (end 47.244 51.816) (width 1) (layer "B.Cu") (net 14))
 (segment (start 47.244 42.926) (end 47.51752 42.926) (width 1) (layer "B.Cu") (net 14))
 (segment (start 47.51752 42.926) (end 49.04401 44.45249) (width 1) (layer "B.Cu") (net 14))
 (segment (start 34.732 45.339) (end 35.179 44.892) (width 1) (layer "B.Cu") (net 12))
 (segment (start 35.179 45.502002) (end 36.268999 46.592001) (width 1) (layer "B.Cu") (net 12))
 (segment (start 40.259 45.502002) (end 40.259 44.892) (width 1) (layer "B.Cu") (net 12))
 (segment (start 35.179 44.892) (end 35.179 45.502002) (width 1) (layer "B.Cu") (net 12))
 (segment (start 30.099 45.339) (end 34.732 45.339) (width 1) (layer "B.Cu") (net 12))
 (segment (start 39.169001 46.592001) (end 40.259 45.502002) (width 1) (layer "B.Cu") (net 12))
 (segment (start 36.268999 46.592001) (end 39.169001 46.592001) (width 1) (layer "B.Cu") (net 12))
 (segment (start 44.969999 43.191999) (end 46.304227 44.526227) (width 1) (layer "B.Cu") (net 13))
 (segment (start 46.304227 44.526227) (end 47.244 45.466) (width 1) (layer "B.Cu") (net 13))
 (segment (start 46.304227 53.416227) (end 47.244 54.356) (width 1) (layer "B.Cu") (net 13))
 (segment (start 45.44399 52.55599) (end 46.304227 53.416227) (width 1) (layer "B.Cu") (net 13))
 (segment (start 47.244 45.466) (end 45.44399 47.26601) (width 1) (layer "B.Cu") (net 13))
 (segment (start 37.719 44.281998) (end 38.808999 43.191999) (width 1) (layer "B.Cu") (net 13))
 (segment (start 37.719 44.892) (end 37.719 44.281998) (width 1) (layer "B.Cu") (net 13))
 (segment (start 45.44399 47.26601) (end 45.44399 52.55599) (width 1) (layer "B.Cu") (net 13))
 (segment (start 38.808999 43.191999) (end 44.969999 43.191999) (width 1) (layer "B.Cu") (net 13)))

